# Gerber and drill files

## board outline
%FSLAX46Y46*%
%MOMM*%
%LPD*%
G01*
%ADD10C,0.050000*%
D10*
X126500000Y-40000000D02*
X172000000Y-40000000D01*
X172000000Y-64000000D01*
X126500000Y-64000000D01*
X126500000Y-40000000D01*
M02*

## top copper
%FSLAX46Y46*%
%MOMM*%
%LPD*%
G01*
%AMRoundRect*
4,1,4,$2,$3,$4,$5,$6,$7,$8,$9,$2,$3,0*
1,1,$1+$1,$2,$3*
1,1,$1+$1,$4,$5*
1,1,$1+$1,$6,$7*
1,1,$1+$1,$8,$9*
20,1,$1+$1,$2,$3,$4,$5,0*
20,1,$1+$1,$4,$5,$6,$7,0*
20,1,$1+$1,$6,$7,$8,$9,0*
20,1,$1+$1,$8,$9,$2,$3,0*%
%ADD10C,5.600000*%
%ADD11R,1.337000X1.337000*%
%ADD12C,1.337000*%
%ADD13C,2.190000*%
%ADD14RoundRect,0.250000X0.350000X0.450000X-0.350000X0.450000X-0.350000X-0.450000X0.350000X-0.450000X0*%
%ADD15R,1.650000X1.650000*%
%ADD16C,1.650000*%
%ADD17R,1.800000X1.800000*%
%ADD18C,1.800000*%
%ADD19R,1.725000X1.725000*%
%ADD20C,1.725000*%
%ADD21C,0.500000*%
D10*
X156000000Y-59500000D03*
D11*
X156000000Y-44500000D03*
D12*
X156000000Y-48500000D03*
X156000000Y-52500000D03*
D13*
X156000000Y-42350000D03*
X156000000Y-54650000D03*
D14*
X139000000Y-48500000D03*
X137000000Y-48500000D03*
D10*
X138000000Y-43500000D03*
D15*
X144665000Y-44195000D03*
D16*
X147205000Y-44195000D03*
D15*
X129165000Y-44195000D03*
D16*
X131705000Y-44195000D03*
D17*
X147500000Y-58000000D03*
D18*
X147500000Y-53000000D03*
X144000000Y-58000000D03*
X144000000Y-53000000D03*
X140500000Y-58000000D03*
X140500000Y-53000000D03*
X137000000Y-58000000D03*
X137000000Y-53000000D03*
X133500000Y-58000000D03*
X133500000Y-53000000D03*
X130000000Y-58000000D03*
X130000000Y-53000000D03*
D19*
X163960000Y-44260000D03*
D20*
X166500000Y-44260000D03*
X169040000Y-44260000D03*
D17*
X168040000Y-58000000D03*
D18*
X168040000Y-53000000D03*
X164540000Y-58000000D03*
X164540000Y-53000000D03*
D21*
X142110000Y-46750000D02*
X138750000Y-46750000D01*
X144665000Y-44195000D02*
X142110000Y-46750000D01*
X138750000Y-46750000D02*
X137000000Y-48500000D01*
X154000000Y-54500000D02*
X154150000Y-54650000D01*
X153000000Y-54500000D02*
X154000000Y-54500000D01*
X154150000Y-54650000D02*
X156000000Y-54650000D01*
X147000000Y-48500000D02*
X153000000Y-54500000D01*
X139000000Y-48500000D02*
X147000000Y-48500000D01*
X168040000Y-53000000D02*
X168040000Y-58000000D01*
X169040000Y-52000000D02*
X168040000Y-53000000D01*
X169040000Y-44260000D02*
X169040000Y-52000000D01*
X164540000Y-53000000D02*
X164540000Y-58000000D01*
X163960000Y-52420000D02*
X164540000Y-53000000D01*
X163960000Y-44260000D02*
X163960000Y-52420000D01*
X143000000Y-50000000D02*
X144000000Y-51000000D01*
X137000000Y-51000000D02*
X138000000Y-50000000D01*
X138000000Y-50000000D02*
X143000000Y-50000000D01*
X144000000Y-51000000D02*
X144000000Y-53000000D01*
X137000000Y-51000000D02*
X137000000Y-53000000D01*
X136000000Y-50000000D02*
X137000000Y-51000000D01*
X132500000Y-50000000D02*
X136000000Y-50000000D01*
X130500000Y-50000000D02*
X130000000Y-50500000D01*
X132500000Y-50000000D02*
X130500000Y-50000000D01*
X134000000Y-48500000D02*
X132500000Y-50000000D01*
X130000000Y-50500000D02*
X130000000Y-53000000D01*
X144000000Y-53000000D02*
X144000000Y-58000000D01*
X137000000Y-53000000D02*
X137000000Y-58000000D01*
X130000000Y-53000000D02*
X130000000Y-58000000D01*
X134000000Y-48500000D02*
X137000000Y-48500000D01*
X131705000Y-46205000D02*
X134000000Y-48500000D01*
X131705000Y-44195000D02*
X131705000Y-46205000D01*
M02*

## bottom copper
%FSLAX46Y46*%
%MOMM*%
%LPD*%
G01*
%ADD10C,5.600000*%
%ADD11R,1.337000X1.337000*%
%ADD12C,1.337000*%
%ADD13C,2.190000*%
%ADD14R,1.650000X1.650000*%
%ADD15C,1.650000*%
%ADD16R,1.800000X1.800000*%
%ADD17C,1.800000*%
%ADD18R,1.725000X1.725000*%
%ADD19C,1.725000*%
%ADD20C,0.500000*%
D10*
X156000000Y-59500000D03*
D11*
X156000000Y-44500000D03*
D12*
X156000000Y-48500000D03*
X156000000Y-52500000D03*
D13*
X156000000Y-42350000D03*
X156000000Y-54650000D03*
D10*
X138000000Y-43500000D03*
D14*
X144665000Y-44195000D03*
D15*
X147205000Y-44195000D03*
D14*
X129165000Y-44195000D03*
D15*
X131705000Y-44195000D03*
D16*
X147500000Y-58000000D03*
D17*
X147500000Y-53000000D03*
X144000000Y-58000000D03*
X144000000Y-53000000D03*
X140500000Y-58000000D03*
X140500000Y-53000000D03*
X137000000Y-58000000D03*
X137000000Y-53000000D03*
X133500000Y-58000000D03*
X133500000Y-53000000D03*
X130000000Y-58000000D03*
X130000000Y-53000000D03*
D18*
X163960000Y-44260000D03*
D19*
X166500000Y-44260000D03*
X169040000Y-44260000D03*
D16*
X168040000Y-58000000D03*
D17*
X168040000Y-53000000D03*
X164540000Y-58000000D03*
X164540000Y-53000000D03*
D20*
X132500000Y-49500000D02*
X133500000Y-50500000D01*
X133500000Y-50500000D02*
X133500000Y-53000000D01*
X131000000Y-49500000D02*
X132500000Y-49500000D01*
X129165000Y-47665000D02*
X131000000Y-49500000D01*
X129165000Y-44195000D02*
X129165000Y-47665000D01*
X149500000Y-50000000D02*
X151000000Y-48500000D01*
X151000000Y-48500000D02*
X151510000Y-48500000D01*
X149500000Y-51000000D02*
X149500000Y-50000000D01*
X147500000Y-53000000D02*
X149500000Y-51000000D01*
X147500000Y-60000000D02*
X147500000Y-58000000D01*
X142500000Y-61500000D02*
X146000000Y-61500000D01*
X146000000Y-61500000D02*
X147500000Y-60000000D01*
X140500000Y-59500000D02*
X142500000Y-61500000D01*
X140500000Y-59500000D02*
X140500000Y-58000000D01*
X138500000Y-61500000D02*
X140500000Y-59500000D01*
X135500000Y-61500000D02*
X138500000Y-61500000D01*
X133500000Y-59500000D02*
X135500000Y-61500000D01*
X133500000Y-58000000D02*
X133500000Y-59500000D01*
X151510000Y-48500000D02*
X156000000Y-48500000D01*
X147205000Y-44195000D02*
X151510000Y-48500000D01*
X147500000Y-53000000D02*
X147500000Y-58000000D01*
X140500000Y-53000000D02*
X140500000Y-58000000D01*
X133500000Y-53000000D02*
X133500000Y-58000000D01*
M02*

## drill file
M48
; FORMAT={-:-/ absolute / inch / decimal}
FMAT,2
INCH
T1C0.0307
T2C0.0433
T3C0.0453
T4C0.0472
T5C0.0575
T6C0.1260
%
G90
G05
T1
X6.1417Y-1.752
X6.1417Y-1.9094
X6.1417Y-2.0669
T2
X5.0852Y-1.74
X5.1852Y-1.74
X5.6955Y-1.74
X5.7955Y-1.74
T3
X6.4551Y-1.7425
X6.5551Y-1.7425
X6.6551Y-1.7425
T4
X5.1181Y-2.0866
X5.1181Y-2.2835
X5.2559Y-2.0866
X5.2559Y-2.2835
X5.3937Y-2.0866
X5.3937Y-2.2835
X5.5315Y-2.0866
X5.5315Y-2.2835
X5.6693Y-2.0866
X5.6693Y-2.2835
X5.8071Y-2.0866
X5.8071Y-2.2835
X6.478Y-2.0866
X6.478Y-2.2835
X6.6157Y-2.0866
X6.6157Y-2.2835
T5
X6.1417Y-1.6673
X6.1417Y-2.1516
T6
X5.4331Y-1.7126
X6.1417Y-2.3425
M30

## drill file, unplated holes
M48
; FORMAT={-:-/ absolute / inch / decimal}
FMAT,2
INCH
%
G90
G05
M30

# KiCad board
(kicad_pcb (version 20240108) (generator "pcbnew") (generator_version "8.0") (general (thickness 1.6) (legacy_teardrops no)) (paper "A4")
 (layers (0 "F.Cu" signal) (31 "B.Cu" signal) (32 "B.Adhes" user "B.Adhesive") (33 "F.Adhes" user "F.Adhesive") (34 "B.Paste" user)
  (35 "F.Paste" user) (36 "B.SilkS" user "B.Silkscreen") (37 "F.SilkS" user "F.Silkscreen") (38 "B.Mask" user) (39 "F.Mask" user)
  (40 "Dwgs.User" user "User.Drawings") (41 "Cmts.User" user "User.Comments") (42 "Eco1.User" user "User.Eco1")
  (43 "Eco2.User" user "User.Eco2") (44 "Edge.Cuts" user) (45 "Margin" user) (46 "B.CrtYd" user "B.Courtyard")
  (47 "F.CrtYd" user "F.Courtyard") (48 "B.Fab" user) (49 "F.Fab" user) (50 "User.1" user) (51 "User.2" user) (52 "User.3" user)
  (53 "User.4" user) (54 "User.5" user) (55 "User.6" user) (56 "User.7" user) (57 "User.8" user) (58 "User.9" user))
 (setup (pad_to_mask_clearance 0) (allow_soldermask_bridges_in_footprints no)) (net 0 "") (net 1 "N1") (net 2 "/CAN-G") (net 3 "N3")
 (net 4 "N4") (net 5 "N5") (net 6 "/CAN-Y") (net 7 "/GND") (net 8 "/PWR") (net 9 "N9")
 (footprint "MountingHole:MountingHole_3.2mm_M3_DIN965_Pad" (layer "F.Cu") (at 156 59.5)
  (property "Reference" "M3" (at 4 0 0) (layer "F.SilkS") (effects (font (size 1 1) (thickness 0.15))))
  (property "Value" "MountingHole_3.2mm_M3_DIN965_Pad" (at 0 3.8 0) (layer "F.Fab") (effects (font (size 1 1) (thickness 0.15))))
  (pad "1" thru_hole circle (at 0 0) (size 5.6 5.6) (drill 3.2) (layers "*.Cu" "*.Mask") (remove_unused_layers no)))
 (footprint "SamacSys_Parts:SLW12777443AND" (layer "F.Cu") (at 156 44.5 -90)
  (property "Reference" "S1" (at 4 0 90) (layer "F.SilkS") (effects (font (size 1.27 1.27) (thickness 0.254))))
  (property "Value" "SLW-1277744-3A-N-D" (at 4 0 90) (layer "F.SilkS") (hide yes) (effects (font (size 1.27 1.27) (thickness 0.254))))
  (pad "1" thru_hole rect (at 0 0) (size 1.337 1.337) (drill 0.78) (layers "*.Cu" "*.Mask" "F.SilkS") (remove_unused_layers no) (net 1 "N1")
   (thermal_bridge_angle 45))
  (pad "2" thru_hole circle (at 4 0) (size 1.337 1.337) (drill 0.78) (layers "*.Cu" "*.Mask" "F.SilkS") (remove_unused_layers no)
   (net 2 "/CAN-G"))
  (pad "3" thru_hole circle (at 8 0) (size 1.337 1.337) (drill 0.78) (layers "*.Cu" "*.Mask" "F.SilkS") (remove_unused_layers no)
   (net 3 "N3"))
  (pad "4" thru_hole circle (at -2.15 0) (size 2.19 2.19) (drill 1.46) (layers "*.Cu" "*.Mask" "F.SilkS") (remove_unused_layers no)
   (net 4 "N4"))
  (pad "5" thru_hole circle (at 10.15 0) (size 2.19 2.19) (drill 1.46) (layers "*.Cu" "*.Mask" "F.SilkS") (remove_unused_layers no)
   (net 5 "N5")))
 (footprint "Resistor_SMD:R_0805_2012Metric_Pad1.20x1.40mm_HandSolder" (layer "F.Cu") (at 138 48.5 180)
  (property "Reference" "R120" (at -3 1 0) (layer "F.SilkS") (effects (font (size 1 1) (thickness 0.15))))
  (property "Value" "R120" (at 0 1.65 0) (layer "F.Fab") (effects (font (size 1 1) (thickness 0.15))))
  (pad "1" smd roundrect (at -1 0 180) (size 1.2 1.4) (layers "F.Cu" "F.Paste" "F.Mask") (roundrect_rratio 0.208333) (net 5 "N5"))
  (pad "2" smd roundrect (at 1 0 180) (size 1.2 1.4) (layers "F.Cu" "F.Paste" "F.Mask") (roundrect_rratio 0.208333) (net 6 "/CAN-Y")))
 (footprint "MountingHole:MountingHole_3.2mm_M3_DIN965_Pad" (layer "F.Cu") (at 138 43.5)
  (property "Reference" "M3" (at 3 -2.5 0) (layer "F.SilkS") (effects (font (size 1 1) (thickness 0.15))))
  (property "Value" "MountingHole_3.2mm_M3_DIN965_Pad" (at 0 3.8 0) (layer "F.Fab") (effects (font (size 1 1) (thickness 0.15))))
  (pad "1" thru_hole circle (at 0 0) (size 5.6 5.6) (drill 3.2) (layers "*.Cu" "*.Mask") (remove_unused_layers no)))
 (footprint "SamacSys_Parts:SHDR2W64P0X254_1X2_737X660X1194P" (layer "F.Cu") (at 144.665 44.195)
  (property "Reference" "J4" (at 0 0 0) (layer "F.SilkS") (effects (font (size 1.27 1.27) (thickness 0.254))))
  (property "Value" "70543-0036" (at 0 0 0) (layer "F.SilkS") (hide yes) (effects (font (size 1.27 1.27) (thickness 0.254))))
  (pad "1" thru_hole rect (at 0 0 90) (size 1.65 1.65) (drill 1.1) (layers "*.Cu" "*.Mask" "F.SilkS") (remove_unused_layers no)
   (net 6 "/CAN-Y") (thermal_bridge_angle 45))
  (pad "2" thru_hole circle (at 2.54 0 90) (size 1.65 1.65) (drill 1.1) (layers "*.Cu" "*.Mask" "F.SilkS") (remove_unused_layers no)
   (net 2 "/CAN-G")))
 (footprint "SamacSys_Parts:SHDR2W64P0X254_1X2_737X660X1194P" (layer "F.Cu") (at 129.165 44.195)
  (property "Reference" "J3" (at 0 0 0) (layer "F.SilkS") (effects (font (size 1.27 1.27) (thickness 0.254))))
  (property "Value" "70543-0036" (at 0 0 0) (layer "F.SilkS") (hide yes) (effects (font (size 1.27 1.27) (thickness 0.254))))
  (pad "1" thru_hole rect (at 0 0 90) (size 1.65 1.65) (drill 1.1) (layers "*.Cu" "*.Mask" "F.SilkS") (remove_unused_layers no)
   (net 2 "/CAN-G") (thermal_bridge_angle 45))
  (pad "2" thru_hole circle (at 2.54 0 90) (size 1.65 1.65) (drill 1.1) (layers "*.Cu" "*.Mask" "F.SilkS") (remove_unused_layers no)
   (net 6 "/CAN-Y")))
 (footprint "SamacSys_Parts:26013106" (layer "F.Cu") (at 147.5 58 180)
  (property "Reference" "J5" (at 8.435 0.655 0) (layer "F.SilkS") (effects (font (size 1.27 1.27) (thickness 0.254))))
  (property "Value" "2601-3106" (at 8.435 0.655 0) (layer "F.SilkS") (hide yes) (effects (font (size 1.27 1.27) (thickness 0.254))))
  (pad "1" thru_hole rect (at 0 0 270) (size 1.8 1.8) (drill 1.2) (layers "*.Cu" "*.Mask" "F.SilkS") (remove_unused_layers no)
   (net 2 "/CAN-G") (thermal_bridge_angle 45))
  (pad "2" thru_hole circle (at 0 5 270) (size 1.8 1.8) (drill 1.2) (layers "*.Cu" "*.Mask" "F.SilkS") (remove_unused_layers no)
   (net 2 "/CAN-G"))
  (pad "3" thru_hole circle (at 3.5 0 270) (size 1.8 1.8) (drill 1.2) (layers "*.Cu" "*.Mask" "F.SilkS") (remove_unused_layers no)
   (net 6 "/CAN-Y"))
  (pad "4" thru_hole circle (at 3.5 5 270) (size 1.8 1.8) (drill 1.2) (layers "*.Cu" "*.Mask" "F.SilkS") (remove_unused_layers no)
   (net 6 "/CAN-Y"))
  (pad "5" thru_hole circle (at 7 0 270) (size 1.8 1.8) (drill 1.2) (layers "*.Cu" "*.Mask" "F.SilkS") (remove_unused_layers no)
   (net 2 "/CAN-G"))
  (pad "6" thru_hole circle (at 7 5 270) (size 1.8 1.8) (drill 1.2) (layers "*.Cu" "*.Mask" "F.SilkS") (remove_unused_layers no)
   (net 2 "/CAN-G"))
  (pad "7" thru_hole circle (at 10.5 0 270) (size 1.8 1.8) (drill 1.2) (layers "*.Cu" "*.Mask" "F.SilkS") (remove_unused_layers no)
   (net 6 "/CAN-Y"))
  (pad "8" thru_hole circle (at 10.5 5 270) (size 1.8 1.8) (drill 1.2) (layers "*.Cu" "*.Mask" "F.SilkS") (remove_unused_layers no)
   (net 6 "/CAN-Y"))
  (pad "9" thru_hole circle (at 14 0 270) (size 1.8 1.8) (drill 1.2) (layers "*.Cu" "*.Mask" "F.SilkS") (remove_unused_layers no)
   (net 2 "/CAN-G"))
  (pad "10" thru_hole circle (at 14 5 270) (size 1.8 1.8) (drill 1.2) (layers "*.Cu" "*.Mask" "F.SilkS") (remove_unused_layers no)
   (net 2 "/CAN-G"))
  (pad "11" thru_hole circle (at 17.5 0 270) (size 1.8 1.8) (drill 1.2) (layers "*.Cu" "*.Mask" "F.SilkS") (remove_unused_layers no)
   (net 6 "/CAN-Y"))
  (pad "12" thru_hole circle (at 17.5 5 270) (size 1.8 1.8) (drill 1.2) (layers "*.Cu" "*.Mask" "F.SilkS") (remove_unused_layers no)
   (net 6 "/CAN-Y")))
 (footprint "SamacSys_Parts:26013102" (layer "F.Cu") (at 168.04 53 180)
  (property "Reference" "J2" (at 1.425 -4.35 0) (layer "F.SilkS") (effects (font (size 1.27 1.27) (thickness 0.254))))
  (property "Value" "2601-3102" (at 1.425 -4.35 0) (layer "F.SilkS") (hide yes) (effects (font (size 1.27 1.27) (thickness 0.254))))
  (pad "1" thru_hole rect (at 0 -5 270) (size 1.8 1.8) (drill 1.2) (layers "*.Cu" "*.Mask" "F.SilkS") (remove_unused_layers no)
   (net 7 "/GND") (thermal_bridge_angle 45))
  (pad "2" thru_hole circle (at 0 0 270) (size 1.8 1.8) (drill 1.2) (layers "*.Cu" "*.Mask" "F.SilkS") (remove_unused_layers no)
   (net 7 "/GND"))
  (pad "3" thru_hole circle (at 3.5 -5 270) (size 1.8 1.8) (drill 1.2) (layers "*.Cu" "*.Mask" "F.SilkS") (remove_unused_layers no)
   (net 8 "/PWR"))
  (pad "4" thru_hole circle (at 3.5 0 270) (size 1.8 1.8) (drill 1.2) (layers "*.Cu" "*.Mask" "F.SilkS") (remove_unused_layers no)
   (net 8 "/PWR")))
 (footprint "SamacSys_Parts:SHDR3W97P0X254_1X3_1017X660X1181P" (layer "F.Cu") (at 163.96 44.26)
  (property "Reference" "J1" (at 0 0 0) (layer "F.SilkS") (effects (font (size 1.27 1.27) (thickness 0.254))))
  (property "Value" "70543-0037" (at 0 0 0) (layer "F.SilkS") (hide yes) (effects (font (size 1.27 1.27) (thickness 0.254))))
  (pad "1" thru_hole rect (at 0 0 90) (size 1.725 1.725) (drill 1.15) (layers "*.Cu" "*.Mask" "F.SilkS") (remove_unused_layers no)
   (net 8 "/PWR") (thermal_bridge_angle 45))
  (pad "2" thru_hole circle (at 2.54 0 90) (size 1.725 1.725) (drill 1.15) (layers "*.Cu" "*.Mask" "F.SilkS") (remove_unused_layers no)
   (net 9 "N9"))
  (pad "3" thru_hole circle (at 5.08 0 90) (size 1.725 1.725) (drill 1.15) (layers "*.Cu" "*.Mask" "F.SilkS") (remove_unused_layers no)
   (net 7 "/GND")))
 (gr_rect (start 126.5 40) (end 172 64) (stroke (width 0.05) (type default)) (fill none) (layer "Edge.Cuts"))
 (segment (start 147.5 53) (end 149.5 51) (width 0.5) (layer "B.Cu") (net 2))
 (segment (start 133.5 58) (end 133.5 59.5) (width 0.5) (layer "B.Cu") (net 2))
 (segment (start 147.205 44.195) (end 151.51 48.5) (width 0.5) (layer "B.Cu") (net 2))
 (segment (start 142.5 61.5) (end 146 61.5) (width 0.5) (layer "B.Cu") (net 2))
 (segment (start 146 61.5) (end 147.5 60) (width 0.5) (layer "B.Cu") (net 2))
 (segment (start 133.5 53) (end 133.5 58) (width 0.5) (layer "B.Cu") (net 2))
 (segment (start 149.5 50) (end 151 48.5) (width 0.5) (layer "B.Cu") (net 2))
 (segment (start 132.5 49.5) (end 133.5 50.5) (width 0.5) (layer "B.Cu") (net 2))
 (segment (start 140.5 59.5) (end 140.5 58) (width 0.5) (layer "B.Cu") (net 2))
 (segment (start 140.5 59.5) (end 142.5 61.5) (width 0.5) (layer "B.Cu") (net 2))
 (segment (start 133.5 59.5) (end 135.5 61.5) (width 0.5) (layer "B.Cu") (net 2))
 (segment (start 147.5 53) (end 147.5 58) (width 0.5) (layer "B.Cu") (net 2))
 (segment (start 129.165 47.665) (end 131 49.5) (width 0.5) (layer "B.Cu") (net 2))
 (segment (start 147.5 60) (end 147.5 58) (width 0.5) (layer "B.Cu") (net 2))
 (segment (start 149.5 51) (end 149.5 50) (width 0.5) (layer "B.Cu") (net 2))
 (segment (start 151.51 48.5) (end 156 48.5) (width 0.5) (layer "B.Cu") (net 2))
 (segment (start 140.5 53) (end 140.5 58) (width 0.5) (layer "B.Cu") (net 2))
 (segment (start 129.165 44.195) (end 129.165 47.665) (width 0.5) (layer "B.Cu") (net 2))
 (segment (start 131 49.5) (end 132.5 49.5) (width 0.5) (layer "B.Cu") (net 2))
 (segment (start 138.5 61.5) (end 140.5 59.5) (width 0.5) (layer "B.Cu") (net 2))
 (segment (start 135.5 61.5) (end 138.5 61.5) (width 0.5) (layer "B.Cu") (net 2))
 (segment (start 133.5 50.5) (end 133.5 53) (width 0.5) (layer "B.Cu") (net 2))
 (segment (start 151 48.5) (end 151.51 48.5) (width 0.5) (layer "B.Cu") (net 2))
 (segment (start 144.665 44.195) (end 142.11 46.75) (width 0.5) (layer "F.Cu") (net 6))
 (segment (start 138.75 46.75) (end 137 48.5) (width 0.5) (layer "F.Cu") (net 6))
 (segment (start 144 51) (end 144 53) (width 0.5) (layer "F.Cu") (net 6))
 (segment (start 144 53) (end 144 58) (width 0.5) (layer "F.Cu") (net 6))
 (segment (start 130 53) (end 130 58) (width 0.5) (layer "F.Cu") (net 6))
 (segment (start 138 50) (end 143 50) (width 0.5) (layer "F.Cu") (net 6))
 (segment (start 134 48.5) (end 132.5 50) (width 0.5) (layer "F.Cu") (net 6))
 (segment (start 130.5 50) (end 130 50.5) (width 0.5) (layer "F.Cu") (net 6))
 (segment (start 137 51) (end 137 53) (width 0.5) (layer "F.Cu") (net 6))
 (segment (start 132.5 50) (end 136 50) (width 0.5) (layer "F.Cu") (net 6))
 (segment (start 137 53) (end 137 58) (width 0.5) (layer "F.Cu") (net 6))
 (segment (start 130 50.5) (end 130 53) (width 0.5) (layer "F.Cu") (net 6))
 (segment (start 131.705 44.195) (end 131.705 46.205) (width 0.5) (layer "F.Cu") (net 6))
 (segment (start 131.705 46.205) (end 134 48.5) (width 0.5) (layer "F.Cu") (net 6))
 (segment (start 142.11 46.75) (end 138.75 46.75) (width 0.5) (layer "F.Cu") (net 6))
 (segment (start 136 50) (end 137 51) (width 0.5) (layer "F.Cu") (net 6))
 (segment (start 132.5 50) (end 130.5 50) (width 0.5) (layer "F.Cu") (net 6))
 (segment (start 134 48.5) (end 137 48.5) (width 0.5) (layer "F.Cu") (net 6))
 (segment (start 137 51) (end 138 50) (width 0.5) (layer "F.Cu") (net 6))
 (segment (start 143 50) (end 144 51) (width 0.5) (layer "F.Cu") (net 6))
 (segment (start 169.04 52) (end 168.04 53) (width 0.5) (layer "F.Cu") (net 7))
 (segment (start 169.04 44.26) (end 169.04 52) (width 0.5) (layer "F.Cu") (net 7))
 (segment (start 168.04 53) (end 168.04 58) (width 0.5) (layer "F.Cu") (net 7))
 (segment (start 163.96 44.26) (end 163.96 52.42) (width 0.5) (layer "F.Cu") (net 8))
 (segment (start 163.96 52.42) (end 164.54 53) (width 0.5) (layer "F.Cu") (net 8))
 (segment (start 164.54 53) (end 164.54 58) (width 0.5) (layer "F.Cu") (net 8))
 (segment (start 153 54.5) (end 154 54.5) (width 0.5) (layer "F.Cu") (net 5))
 (segment (start 154 54.5) (end 154.15 54.65) (width 0.5) (layer "F.Cu") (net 5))
 (segment (start 147 48.5) (end 153 54.5) (width 0.5) (layer "F.Cu") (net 5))
 (segment (start 154.15 54.65) (end 156 54.65) (width 0.5) (layer "F.Cu") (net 5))
 (segment (start 139 48.5) (end 147 48.5) (width 0.5) (layer "F.Cu") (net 5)))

